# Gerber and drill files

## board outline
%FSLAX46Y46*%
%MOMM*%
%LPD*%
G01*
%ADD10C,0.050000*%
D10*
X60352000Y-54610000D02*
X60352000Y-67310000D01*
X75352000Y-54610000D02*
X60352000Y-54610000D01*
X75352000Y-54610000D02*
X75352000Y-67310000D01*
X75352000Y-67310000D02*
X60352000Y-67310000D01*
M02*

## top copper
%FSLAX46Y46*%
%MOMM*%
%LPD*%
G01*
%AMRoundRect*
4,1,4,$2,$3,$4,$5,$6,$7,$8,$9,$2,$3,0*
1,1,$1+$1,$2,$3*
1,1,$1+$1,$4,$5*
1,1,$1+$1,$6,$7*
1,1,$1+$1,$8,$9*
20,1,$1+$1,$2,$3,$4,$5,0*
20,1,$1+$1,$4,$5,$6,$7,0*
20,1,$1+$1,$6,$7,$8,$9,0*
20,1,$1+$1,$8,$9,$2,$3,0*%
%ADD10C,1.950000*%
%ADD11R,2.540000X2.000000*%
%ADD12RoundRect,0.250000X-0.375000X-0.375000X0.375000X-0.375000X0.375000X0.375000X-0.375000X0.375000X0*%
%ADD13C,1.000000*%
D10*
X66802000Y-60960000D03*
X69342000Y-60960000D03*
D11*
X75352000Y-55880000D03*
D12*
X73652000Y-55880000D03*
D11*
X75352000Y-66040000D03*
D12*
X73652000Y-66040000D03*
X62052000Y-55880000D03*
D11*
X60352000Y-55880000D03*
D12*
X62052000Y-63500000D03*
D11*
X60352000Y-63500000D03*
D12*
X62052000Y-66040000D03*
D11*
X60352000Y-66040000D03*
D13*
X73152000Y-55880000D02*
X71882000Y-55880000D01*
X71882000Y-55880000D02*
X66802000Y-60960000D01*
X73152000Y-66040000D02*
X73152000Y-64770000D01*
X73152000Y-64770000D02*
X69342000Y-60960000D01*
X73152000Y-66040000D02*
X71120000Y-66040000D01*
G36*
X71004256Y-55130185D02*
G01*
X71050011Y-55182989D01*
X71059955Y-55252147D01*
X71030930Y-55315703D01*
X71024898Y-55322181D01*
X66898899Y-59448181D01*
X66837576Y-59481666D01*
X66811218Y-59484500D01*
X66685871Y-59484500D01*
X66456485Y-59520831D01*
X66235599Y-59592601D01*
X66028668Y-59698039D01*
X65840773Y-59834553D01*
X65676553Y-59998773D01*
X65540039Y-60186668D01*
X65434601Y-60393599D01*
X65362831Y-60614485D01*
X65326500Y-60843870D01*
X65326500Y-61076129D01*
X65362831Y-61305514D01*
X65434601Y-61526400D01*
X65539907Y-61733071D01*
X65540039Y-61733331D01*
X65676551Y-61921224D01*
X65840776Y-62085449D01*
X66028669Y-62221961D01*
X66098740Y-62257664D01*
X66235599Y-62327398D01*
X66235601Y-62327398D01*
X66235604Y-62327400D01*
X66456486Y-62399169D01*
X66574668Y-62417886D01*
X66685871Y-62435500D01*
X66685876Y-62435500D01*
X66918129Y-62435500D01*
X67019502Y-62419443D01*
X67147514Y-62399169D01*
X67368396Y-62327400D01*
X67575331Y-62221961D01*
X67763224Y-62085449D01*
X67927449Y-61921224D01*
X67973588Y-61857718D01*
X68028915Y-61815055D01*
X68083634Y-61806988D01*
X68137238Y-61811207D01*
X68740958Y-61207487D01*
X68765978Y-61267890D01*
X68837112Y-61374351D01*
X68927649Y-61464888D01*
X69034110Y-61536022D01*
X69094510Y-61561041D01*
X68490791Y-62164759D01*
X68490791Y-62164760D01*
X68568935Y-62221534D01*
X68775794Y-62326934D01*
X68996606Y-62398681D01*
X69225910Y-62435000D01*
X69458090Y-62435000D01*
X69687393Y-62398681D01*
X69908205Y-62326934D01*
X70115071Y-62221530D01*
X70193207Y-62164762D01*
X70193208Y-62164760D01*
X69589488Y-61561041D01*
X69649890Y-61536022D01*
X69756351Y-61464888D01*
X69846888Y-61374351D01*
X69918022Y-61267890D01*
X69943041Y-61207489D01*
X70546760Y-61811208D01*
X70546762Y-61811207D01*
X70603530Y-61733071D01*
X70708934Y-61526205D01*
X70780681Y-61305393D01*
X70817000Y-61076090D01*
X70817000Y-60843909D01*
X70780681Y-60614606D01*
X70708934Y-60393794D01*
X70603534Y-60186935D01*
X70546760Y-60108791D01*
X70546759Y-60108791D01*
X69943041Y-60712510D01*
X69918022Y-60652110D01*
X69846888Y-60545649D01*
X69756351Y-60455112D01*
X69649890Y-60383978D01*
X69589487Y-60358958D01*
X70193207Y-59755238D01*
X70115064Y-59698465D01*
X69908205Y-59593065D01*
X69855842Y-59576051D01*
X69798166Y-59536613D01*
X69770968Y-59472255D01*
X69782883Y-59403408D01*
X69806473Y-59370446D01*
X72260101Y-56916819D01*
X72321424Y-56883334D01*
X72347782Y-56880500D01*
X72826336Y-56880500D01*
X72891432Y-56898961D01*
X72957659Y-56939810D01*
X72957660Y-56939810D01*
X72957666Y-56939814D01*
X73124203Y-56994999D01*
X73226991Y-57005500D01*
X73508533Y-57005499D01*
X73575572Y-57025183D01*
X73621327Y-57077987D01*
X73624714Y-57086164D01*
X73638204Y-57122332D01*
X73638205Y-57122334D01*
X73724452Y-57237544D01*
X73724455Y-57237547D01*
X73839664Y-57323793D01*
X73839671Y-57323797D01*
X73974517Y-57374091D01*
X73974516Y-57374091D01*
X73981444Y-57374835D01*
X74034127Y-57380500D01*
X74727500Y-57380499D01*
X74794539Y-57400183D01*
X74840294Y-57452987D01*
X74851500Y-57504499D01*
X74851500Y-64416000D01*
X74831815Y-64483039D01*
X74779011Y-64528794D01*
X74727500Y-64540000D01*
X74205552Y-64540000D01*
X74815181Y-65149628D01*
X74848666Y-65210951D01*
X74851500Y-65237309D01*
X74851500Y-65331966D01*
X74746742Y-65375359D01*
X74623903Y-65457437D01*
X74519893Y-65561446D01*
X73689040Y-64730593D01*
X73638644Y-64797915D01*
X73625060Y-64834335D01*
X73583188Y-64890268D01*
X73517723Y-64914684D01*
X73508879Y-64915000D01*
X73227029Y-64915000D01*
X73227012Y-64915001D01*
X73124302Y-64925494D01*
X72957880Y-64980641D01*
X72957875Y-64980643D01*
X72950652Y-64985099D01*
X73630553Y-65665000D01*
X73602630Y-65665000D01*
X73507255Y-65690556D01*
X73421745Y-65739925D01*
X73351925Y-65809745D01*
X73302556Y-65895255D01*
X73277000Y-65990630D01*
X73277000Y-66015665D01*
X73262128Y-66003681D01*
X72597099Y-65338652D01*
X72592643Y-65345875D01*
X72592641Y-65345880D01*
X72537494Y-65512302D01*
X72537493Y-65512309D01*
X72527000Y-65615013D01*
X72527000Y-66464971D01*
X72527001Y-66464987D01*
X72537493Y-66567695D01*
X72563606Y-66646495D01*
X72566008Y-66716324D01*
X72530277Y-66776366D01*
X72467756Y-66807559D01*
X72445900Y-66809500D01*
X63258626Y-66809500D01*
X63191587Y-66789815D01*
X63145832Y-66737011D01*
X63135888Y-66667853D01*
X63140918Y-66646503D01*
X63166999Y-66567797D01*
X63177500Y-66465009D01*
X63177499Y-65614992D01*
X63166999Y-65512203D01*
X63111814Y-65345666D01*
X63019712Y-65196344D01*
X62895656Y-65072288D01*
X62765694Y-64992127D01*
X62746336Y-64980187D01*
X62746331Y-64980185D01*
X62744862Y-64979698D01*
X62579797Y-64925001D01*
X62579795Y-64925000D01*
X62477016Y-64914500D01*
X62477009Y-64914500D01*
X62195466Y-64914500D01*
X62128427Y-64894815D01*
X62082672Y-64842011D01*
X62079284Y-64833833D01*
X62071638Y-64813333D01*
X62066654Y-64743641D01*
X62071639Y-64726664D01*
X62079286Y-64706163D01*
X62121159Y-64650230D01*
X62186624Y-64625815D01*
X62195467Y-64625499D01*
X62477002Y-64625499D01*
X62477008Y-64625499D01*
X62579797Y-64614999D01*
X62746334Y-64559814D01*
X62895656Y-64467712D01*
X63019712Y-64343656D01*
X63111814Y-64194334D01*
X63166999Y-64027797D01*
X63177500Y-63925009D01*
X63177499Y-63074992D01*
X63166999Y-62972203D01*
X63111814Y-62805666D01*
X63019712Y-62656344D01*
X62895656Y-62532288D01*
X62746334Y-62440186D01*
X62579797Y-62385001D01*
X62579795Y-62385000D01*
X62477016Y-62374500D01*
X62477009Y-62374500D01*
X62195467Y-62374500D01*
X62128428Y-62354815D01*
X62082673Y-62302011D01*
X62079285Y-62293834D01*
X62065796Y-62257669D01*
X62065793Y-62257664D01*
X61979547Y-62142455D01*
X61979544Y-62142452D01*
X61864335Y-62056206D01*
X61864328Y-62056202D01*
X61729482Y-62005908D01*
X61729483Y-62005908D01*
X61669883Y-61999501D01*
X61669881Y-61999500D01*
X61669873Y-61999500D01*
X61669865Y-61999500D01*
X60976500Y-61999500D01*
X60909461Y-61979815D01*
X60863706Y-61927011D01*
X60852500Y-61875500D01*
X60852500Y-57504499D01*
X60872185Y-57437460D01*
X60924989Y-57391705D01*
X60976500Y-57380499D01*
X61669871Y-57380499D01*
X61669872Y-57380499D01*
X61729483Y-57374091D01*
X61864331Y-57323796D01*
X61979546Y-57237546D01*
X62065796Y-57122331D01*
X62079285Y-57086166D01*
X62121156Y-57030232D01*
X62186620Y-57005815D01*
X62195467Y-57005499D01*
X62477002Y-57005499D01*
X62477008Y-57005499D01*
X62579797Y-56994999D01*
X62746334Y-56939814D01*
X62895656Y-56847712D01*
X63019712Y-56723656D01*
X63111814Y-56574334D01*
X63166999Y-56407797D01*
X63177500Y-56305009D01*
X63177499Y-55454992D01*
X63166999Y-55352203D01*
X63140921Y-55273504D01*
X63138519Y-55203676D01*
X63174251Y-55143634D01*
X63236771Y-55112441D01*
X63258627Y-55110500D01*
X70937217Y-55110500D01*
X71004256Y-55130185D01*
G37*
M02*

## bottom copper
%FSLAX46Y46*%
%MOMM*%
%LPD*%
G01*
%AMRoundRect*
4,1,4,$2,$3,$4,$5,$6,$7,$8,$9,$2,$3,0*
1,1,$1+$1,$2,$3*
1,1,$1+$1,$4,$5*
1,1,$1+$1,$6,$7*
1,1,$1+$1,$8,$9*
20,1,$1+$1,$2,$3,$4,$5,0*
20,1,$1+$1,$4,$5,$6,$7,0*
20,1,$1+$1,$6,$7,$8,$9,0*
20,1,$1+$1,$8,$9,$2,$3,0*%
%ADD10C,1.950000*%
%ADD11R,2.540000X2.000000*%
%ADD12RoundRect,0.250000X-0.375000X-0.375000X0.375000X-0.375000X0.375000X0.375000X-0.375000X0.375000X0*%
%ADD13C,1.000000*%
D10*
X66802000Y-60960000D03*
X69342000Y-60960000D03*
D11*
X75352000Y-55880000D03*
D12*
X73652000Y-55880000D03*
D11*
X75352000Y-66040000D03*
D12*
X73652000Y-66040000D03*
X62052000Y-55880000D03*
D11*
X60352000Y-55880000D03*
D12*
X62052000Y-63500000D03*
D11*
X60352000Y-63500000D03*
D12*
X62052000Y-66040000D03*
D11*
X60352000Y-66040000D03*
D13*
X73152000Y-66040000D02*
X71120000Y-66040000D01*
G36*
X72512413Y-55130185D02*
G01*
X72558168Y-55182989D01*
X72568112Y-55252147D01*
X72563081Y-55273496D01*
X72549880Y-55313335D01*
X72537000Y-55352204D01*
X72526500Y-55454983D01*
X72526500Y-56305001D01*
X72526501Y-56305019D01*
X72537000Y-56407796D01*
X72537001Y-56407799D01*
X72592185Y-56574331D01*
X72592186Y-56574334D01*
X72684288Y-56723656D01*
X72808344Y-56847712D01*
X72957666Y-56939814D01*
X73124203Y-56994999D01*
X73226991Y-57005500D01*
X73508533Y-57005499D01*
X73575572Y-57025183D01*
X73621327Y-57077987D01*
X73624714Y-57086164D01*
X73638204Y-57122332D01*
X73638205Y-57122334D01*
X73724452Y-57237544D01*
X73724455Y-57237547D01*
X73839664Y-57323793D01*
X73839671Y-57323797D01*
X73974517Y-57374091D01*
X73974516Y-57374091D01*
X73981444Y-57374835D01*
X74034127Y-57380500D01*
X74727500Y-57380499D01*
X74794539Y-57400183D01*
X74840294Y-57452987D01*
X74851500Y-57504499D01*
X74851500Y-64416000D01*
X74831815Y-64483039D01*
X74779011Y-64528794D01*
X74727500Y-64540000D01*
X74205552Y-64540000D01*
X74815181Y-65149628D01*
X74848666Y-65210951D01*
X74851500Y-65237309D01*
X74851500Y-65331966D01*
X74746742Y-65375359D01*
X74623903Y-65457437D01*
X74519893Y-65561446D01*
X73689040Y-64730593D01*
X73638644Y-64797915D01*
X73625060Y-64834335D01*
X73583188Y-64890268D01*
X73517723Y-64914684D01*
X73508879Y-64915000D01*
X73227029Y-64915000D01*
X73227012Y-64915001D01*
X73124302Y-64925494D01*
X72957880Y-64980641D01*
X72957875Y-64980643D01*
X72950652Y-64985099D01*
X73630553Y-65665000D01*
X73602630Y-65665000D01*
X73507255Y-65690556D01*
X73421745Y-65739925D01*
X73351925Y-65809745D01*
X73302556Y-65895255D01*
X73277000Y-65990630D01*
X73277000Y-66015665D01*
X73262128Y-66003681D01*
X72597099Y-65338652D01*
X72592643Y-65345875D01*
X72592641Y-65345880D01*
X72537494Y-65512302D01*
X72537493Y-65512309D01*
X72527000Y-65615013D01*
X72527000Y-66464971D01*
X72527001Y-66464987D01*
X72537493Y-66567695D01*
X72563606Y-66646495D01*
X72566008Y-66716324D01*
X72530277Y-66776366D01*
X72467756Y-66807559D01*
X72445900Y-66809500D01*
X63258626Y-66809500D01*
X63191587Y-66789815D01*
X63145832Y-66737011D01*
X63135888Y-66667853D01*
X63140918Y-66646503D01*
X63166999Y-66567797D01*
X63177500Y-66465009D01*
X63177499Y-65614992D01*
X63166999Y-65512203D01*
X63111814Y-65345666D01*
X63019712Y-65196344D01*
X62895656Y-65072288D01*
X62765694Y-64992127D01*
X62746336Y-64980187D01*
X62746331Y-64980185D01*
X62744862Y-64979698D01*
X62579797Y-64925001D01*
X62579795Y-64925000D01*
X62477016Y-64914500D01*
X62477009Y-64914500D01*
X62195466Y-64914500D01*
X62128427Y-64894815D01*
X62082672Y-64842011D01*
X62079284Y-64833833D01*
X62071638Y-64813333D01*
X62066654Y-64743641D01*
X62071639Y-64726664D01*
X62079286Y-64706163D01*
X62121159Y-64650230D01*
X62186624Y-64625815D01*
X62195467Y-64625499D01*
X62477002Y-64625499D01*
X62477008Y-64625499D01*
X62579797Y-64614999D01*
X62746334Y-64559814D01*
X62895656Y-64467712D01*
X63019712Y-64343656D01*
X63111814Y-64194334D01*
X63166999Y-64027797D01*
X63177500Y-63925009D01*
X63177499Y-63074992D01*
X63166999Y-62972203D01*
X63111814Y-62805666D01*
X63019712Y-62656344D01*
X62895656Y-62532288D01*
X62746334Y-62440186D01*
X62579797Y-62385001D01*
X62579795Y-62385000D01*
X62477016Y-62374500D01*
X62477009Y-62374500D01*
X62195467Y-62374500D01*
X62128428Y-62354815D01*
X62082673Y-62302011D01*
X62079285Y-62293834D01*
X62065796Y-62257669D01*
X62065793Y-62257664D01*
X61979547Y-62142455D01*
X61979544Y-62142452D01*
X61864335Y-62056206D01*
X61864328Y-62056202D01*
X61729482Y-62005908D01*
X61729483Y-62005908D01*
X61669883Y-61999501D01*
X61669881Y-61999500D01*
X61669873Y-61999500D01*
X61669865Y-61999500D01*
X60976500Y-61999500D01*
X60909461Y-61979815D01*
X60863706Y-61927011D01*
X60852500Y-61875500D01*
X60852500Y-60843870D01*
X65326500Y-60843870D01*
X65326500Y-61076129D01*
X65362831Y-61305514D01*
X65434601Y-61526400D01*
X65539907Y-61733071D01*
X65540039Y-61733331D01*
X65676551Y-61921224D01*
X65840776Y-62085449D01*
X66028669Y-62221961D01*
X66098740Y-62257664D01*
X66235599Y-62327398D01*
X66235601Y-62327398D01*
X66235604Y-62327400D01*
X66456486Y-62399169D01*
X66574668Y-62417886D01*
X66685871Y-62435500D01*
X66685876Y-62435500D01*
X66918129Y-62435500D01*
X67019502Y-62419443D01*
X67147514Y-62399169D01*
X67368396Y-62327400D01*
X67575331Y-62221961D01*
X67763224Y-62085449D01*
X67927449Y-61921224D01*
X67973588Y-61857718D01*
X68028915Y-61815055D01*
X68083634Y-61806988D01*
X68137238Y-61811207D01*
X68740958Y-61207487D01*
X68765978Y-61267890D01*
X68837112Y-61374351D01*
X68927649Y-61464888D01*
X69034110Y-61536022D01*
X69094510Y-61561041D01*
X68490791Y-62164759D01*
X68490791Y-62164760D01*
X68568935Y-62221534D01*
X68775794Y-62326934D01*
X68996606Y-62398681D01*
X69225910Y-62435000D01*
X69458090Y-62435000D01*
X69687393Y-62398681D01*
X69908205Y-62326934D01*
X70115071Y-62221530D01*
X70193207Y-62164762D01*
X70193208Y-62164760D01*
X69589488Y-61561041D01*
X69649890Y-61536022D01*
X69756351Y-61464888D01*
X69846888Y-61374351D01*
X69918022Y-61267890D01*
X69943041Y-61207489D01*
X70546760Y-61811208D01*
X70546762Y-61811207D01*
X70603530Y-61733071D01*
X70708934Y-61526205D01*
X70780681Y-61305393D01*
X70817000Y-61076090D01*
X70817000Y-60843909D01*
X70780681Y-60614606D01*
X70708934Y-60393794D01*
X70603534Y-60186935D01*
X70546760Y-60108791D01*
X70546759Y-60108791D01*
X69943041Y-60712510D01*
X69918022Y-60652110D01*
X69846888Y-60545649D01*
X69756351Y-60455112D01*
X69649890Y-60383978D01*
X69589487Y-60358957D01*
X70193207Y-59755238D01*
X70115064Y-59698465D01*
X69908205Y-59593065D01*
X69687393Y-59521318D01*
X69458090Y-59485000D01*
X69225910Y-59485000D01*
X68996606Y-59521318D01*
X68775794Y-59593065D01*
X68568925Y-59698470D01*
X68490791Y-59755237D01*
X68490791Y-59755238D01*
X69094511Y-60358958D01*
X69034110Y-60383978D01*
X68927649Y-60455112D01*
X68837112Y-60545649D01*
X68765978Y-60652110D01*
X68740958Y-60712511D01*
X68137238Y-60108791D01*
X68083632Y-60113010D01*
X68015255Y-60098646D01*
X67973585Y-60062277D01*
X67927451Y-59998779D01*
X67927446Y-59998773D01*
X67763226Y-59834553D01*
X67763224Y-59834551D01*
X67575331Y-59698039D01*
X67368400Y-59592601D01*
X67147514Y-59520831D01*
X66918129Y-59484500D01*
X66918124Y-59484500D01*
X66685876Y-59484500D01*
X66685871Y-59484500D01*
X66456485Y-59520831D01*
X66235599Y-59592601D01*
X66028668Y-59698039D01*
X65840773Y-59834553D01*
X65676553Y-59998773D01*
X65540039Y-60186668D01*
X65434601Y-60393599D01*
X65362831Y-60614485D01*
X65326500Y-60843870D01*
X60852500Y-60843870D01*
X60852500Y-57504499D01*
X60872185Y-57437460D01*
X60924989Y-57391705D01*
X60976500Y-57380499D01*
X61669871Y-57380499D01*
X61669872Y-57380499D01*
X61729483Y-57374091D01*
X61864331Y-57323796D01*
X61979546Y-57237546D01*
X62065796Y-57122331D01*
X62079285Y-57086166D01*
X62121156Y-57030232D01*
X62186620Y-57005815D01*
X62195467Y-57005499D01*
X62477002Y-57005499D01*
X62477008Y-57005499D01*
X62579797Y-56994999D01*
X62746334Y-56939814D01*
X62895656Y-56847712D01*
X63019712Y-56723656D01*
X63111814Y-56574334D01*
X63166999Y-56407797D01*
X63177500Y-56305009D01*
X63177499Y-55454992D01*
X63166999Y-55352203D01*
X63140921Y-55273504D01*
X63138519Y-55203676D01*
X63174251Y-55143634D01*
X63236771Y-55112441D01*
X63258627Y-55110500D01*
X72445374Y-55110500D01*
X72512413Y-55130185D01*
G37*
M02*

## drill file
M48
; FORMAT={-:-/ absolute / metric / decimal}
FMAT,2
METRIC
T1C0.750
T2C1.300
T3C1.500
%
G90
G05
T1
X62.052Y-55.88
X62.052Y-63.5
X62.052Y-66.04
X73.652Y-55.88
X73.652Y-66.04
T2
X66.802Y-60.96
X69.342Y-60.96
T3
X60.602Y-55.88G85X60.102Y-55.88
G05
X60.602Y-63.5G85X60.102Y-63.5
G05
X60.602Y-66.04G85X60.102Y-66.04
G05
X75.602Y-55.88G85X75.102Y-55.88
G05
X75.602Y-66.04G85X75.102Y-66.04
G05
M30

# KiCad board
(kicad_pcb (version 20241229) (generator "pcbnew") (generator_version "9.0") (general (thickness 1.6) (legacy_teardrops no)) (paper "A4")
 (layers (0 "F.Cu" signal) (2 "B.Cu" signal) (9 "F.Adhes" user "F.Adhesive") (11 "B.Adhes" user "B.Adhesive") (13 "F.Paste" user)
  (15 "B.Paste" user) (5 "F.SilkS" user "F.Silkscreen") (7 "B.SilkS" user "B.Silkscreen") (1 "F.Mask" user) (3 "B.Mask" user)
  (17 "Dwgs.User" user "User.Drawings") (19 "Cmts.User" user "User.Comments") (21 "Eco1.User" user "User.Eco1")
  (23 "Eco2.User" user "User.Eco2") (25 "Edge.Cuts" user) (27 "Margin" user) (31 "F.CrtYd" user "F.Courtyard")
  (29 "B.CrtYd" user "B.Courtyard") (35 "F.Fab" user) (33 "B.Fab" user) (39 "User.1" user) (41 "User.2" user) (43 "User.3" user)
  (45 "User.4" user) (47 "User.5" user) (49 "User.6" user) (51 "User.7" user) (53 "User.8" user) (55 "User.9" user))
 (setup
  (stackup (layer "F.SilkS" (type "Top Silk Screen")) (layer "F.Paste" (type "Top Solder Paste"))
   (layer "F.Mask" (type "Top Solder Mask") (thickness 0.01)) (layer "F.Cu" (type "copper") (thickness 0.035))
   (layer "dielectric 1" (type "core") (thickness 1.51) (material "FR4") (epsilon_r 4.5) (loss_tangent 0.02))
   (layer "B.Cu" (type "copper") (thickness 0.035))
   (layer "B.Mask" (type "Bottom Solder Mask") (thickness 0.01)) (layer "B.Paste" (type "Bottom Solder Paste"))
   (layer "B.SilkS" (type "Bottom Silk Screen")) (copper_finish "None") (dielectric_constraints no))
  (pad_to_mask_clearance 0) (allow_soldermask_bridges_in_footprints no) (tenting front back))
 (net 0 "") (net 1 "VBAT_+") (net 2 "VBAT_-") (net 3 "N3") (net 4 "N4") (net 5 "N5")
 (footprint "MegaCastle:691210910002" (layer "F.Cu") (at 68.072 60.96)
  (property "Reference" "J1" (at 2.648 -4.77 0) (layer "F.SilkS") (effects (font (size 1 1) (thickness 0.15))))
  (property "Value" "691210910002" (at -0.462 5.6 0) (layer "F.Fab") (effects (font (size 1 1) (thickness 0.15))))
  (pad "1" thru_hole circle (at -1.27 0) (size 1.95 1.95) (drill 1.3) (layers "*.Cu" "*.Mask") (remove_unused_layers no) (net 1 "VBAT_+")
   (solder_mask_margin 0.102))
  (pad "2" thru_hole circle (at 1.27 0) (size 1.95 1.95) (drill 1.3) (layers "*.Cu" "*.Mask") (remove_unused_layers no) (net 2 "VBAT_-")
   (solder_mask_margin 0.102)))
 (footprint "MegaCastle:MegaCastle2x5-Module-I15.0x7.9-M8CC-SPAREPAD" (layer "B.Cu") (at 67.852 60.96 180)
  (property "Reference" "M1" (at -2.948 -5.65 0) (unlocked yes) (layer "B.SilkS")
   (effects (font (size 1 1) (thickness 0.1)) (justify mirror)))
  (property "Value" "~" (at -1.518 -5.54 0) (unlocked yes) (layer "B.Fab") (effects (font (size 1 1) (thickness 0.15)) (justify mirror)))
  (fp_line (start 7.5 6.35) (end 7.5 -6.35) (stroke (width 0.05) (type default)) (layer "Edge.Cuts"))
  (fp_line (start -7.5 6.35) (end 7.5 6.35) (stroke (width 0.05) (type default)) (layer "Edge.Cuts"))
  (fp_line (start -7.5 6.35) (end -7.5 -6.35) (stroke (width 0.05) (type default)) (layer "Edge.Cuts"))
  (fp_line (start -7.5 -6.35) (end 7.5 -6.35) (stroke (width 0.05) (type default)) (layer "Edge.Cuts"))
  (pad "1" thru_hole rect (at -7.5 5.08 180) (size 2.54 2) (drill oval 2 1.5) (layers "*.Cu" "*.Mask") (remove_unused_layers no)
   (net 1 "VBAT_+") (thermal_bridge_angle 45))
  (pad "1" thru_hole roundrect (at -5.8 5.08) (size 1.25 1.25) (drill 0.75) (layers "*.Cu" "*.Mask") (remove_unused_layers no)
   (roundrect_rratio 0.2) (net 1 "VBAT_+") (thermal_bridge_angle 45))
  (pad "5" thru_hole rect (at -7.5 -5.08 180) (size 2.54 2) (drill oval 2 1.5) (layers "*.Cu" "*.Mask") (remove_unused_layers no)
   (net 2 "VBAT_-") (thermal_bridge_angle 45))
  (pad "5" thru_hole roundrect (at -5.8 -5.08) (size 1.25 1.25) (drill 0.75) (layers "*.Cu" "*.Mask") (remove_unused_layers no)
   (roundrect_rratio 0.2) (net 2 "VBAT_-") (thermal_bridge_angle 45))
  (pad "6" thru_hole roundrect (at 5.8 5.08) (size 1.25 1.25) (drill 0.75) (layers "*.Cu" "*.Mask") (remove_unused_layers no)
   (roundrect_rratio 0.2) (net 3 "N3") (thermal_bridge_angle 45))
  (pad "6" thru_hole rect (at 7.5 5.08 180) (size 2.54 2) (drill oval 2 1.5) (layers "*.Cu" "*.Mask") (remove_unused_layers no) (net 3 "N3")
   (thermal_bridge_angle 45))
  (pad "9" thru_hole roundrect (at 5.8 -2.54) (size 1.25 1.25) (drill 0.75) (layers "*.Cu" "*.Mask") (remove_unused_layers no)
   (roundrect_rratio 0.2) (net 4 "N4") (thermal_bridge_angle 45))
  (pad "9" thru_hole rect (at 7.5 -2.54 180) (size 2.54 2) (drill oval 2 1.5) (layers "*.Cu" "*.Mask") (remove_unused_layers no)
   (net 4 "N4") (thermal_bridge_angle 45))
  (pad "10" thru_hole roundrect (at 5.8 -5.08) (size 1.25 1.25) (drill 0.75) (layers "*.Cu" "*.Mask") (remove_unused_layers no)
   (roundrect_rratio 0.2) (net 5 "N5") (thermal_bridge_angle 45))
  (pad "10" thru_hole rect (at 7.5 -5.08 180) (size 2.54 2) (drill oval 2 1.5) (layers "*.Cu" "*.Mask") (remove_unused_layers no)
   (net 5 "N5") (thermal_bridge_angle 45))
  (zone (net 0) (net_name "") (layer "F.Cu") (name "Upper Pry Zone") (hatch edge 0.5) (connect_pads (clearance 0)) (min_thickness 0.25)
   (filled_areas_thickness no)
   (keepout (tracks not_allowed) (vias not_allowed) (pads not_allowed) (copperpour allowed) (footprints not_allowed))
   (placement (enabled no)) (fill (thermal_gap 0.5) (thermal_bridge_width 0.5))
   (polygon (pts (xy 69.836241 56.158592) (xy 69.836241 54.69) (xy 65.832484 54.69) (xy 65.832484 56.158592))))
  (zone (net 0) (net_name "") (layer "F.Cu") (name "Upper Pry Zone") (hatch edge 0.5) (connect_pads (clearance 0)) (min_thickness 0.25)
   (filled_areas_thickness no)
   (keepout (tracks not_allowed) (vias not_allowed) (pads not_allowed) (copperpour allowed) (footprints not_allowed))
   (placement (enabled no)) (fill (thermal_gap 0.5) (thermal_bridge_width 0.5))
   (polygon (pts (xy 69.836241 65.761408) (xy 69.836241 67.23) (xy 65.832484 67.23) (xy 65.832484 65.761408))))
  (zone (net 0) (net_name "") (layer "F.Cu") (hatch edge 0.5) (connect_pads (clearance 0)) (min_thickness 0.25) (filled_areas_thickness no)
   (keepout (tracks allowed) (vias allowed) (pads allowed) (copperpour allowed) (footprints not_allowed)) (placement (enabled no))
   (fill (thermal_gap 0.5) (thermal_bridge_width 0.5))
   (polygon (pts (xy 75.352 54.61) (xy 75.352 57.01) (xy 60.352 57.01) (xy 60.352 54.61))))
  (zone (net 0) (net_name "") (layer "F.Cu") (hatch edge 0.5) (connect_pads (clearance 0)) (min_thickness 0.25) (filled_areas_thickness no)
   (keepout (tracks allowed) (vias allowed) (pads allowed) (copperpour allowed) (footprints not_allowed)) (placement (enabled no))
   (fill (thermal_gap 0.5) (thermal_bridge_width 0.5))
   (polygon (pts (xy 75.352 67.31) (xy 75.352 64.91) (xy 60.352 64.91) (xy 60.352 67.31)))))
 (segment (start 73.152 55.88) (end 71.882 55.88) (width 1) (layer "F.Cu") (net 1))
 (segment (start 71.882 55.88) (end 66.802 60.96) (width 1) (layer "F.Cu") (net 1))
 (segment (start 73.152 66.04) (end 73.152 64.77) (width 1) (layer "F.Cu") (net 2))
 (segment (start 73.152 64.77) (end 69.342 60.96) (width 1) (layer "F.Cu") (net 2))
 (segment (start 73.152 66.04) (end 71.12 66.04) (width 1) (layer "F.Cu") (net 2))
 (segment (start 73.152 66.04) (end 71.12 66.04) (width 1) (layer "B.Cu") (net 2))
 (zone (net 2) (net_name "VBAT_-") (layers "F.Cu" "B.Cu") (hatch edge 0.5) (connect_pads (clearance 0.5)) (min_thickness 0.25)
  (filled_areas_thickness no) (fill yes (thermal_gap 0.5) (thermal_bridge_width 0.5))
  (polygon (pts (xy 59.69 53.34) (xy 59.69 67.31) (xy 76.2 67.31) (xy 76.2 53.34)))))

